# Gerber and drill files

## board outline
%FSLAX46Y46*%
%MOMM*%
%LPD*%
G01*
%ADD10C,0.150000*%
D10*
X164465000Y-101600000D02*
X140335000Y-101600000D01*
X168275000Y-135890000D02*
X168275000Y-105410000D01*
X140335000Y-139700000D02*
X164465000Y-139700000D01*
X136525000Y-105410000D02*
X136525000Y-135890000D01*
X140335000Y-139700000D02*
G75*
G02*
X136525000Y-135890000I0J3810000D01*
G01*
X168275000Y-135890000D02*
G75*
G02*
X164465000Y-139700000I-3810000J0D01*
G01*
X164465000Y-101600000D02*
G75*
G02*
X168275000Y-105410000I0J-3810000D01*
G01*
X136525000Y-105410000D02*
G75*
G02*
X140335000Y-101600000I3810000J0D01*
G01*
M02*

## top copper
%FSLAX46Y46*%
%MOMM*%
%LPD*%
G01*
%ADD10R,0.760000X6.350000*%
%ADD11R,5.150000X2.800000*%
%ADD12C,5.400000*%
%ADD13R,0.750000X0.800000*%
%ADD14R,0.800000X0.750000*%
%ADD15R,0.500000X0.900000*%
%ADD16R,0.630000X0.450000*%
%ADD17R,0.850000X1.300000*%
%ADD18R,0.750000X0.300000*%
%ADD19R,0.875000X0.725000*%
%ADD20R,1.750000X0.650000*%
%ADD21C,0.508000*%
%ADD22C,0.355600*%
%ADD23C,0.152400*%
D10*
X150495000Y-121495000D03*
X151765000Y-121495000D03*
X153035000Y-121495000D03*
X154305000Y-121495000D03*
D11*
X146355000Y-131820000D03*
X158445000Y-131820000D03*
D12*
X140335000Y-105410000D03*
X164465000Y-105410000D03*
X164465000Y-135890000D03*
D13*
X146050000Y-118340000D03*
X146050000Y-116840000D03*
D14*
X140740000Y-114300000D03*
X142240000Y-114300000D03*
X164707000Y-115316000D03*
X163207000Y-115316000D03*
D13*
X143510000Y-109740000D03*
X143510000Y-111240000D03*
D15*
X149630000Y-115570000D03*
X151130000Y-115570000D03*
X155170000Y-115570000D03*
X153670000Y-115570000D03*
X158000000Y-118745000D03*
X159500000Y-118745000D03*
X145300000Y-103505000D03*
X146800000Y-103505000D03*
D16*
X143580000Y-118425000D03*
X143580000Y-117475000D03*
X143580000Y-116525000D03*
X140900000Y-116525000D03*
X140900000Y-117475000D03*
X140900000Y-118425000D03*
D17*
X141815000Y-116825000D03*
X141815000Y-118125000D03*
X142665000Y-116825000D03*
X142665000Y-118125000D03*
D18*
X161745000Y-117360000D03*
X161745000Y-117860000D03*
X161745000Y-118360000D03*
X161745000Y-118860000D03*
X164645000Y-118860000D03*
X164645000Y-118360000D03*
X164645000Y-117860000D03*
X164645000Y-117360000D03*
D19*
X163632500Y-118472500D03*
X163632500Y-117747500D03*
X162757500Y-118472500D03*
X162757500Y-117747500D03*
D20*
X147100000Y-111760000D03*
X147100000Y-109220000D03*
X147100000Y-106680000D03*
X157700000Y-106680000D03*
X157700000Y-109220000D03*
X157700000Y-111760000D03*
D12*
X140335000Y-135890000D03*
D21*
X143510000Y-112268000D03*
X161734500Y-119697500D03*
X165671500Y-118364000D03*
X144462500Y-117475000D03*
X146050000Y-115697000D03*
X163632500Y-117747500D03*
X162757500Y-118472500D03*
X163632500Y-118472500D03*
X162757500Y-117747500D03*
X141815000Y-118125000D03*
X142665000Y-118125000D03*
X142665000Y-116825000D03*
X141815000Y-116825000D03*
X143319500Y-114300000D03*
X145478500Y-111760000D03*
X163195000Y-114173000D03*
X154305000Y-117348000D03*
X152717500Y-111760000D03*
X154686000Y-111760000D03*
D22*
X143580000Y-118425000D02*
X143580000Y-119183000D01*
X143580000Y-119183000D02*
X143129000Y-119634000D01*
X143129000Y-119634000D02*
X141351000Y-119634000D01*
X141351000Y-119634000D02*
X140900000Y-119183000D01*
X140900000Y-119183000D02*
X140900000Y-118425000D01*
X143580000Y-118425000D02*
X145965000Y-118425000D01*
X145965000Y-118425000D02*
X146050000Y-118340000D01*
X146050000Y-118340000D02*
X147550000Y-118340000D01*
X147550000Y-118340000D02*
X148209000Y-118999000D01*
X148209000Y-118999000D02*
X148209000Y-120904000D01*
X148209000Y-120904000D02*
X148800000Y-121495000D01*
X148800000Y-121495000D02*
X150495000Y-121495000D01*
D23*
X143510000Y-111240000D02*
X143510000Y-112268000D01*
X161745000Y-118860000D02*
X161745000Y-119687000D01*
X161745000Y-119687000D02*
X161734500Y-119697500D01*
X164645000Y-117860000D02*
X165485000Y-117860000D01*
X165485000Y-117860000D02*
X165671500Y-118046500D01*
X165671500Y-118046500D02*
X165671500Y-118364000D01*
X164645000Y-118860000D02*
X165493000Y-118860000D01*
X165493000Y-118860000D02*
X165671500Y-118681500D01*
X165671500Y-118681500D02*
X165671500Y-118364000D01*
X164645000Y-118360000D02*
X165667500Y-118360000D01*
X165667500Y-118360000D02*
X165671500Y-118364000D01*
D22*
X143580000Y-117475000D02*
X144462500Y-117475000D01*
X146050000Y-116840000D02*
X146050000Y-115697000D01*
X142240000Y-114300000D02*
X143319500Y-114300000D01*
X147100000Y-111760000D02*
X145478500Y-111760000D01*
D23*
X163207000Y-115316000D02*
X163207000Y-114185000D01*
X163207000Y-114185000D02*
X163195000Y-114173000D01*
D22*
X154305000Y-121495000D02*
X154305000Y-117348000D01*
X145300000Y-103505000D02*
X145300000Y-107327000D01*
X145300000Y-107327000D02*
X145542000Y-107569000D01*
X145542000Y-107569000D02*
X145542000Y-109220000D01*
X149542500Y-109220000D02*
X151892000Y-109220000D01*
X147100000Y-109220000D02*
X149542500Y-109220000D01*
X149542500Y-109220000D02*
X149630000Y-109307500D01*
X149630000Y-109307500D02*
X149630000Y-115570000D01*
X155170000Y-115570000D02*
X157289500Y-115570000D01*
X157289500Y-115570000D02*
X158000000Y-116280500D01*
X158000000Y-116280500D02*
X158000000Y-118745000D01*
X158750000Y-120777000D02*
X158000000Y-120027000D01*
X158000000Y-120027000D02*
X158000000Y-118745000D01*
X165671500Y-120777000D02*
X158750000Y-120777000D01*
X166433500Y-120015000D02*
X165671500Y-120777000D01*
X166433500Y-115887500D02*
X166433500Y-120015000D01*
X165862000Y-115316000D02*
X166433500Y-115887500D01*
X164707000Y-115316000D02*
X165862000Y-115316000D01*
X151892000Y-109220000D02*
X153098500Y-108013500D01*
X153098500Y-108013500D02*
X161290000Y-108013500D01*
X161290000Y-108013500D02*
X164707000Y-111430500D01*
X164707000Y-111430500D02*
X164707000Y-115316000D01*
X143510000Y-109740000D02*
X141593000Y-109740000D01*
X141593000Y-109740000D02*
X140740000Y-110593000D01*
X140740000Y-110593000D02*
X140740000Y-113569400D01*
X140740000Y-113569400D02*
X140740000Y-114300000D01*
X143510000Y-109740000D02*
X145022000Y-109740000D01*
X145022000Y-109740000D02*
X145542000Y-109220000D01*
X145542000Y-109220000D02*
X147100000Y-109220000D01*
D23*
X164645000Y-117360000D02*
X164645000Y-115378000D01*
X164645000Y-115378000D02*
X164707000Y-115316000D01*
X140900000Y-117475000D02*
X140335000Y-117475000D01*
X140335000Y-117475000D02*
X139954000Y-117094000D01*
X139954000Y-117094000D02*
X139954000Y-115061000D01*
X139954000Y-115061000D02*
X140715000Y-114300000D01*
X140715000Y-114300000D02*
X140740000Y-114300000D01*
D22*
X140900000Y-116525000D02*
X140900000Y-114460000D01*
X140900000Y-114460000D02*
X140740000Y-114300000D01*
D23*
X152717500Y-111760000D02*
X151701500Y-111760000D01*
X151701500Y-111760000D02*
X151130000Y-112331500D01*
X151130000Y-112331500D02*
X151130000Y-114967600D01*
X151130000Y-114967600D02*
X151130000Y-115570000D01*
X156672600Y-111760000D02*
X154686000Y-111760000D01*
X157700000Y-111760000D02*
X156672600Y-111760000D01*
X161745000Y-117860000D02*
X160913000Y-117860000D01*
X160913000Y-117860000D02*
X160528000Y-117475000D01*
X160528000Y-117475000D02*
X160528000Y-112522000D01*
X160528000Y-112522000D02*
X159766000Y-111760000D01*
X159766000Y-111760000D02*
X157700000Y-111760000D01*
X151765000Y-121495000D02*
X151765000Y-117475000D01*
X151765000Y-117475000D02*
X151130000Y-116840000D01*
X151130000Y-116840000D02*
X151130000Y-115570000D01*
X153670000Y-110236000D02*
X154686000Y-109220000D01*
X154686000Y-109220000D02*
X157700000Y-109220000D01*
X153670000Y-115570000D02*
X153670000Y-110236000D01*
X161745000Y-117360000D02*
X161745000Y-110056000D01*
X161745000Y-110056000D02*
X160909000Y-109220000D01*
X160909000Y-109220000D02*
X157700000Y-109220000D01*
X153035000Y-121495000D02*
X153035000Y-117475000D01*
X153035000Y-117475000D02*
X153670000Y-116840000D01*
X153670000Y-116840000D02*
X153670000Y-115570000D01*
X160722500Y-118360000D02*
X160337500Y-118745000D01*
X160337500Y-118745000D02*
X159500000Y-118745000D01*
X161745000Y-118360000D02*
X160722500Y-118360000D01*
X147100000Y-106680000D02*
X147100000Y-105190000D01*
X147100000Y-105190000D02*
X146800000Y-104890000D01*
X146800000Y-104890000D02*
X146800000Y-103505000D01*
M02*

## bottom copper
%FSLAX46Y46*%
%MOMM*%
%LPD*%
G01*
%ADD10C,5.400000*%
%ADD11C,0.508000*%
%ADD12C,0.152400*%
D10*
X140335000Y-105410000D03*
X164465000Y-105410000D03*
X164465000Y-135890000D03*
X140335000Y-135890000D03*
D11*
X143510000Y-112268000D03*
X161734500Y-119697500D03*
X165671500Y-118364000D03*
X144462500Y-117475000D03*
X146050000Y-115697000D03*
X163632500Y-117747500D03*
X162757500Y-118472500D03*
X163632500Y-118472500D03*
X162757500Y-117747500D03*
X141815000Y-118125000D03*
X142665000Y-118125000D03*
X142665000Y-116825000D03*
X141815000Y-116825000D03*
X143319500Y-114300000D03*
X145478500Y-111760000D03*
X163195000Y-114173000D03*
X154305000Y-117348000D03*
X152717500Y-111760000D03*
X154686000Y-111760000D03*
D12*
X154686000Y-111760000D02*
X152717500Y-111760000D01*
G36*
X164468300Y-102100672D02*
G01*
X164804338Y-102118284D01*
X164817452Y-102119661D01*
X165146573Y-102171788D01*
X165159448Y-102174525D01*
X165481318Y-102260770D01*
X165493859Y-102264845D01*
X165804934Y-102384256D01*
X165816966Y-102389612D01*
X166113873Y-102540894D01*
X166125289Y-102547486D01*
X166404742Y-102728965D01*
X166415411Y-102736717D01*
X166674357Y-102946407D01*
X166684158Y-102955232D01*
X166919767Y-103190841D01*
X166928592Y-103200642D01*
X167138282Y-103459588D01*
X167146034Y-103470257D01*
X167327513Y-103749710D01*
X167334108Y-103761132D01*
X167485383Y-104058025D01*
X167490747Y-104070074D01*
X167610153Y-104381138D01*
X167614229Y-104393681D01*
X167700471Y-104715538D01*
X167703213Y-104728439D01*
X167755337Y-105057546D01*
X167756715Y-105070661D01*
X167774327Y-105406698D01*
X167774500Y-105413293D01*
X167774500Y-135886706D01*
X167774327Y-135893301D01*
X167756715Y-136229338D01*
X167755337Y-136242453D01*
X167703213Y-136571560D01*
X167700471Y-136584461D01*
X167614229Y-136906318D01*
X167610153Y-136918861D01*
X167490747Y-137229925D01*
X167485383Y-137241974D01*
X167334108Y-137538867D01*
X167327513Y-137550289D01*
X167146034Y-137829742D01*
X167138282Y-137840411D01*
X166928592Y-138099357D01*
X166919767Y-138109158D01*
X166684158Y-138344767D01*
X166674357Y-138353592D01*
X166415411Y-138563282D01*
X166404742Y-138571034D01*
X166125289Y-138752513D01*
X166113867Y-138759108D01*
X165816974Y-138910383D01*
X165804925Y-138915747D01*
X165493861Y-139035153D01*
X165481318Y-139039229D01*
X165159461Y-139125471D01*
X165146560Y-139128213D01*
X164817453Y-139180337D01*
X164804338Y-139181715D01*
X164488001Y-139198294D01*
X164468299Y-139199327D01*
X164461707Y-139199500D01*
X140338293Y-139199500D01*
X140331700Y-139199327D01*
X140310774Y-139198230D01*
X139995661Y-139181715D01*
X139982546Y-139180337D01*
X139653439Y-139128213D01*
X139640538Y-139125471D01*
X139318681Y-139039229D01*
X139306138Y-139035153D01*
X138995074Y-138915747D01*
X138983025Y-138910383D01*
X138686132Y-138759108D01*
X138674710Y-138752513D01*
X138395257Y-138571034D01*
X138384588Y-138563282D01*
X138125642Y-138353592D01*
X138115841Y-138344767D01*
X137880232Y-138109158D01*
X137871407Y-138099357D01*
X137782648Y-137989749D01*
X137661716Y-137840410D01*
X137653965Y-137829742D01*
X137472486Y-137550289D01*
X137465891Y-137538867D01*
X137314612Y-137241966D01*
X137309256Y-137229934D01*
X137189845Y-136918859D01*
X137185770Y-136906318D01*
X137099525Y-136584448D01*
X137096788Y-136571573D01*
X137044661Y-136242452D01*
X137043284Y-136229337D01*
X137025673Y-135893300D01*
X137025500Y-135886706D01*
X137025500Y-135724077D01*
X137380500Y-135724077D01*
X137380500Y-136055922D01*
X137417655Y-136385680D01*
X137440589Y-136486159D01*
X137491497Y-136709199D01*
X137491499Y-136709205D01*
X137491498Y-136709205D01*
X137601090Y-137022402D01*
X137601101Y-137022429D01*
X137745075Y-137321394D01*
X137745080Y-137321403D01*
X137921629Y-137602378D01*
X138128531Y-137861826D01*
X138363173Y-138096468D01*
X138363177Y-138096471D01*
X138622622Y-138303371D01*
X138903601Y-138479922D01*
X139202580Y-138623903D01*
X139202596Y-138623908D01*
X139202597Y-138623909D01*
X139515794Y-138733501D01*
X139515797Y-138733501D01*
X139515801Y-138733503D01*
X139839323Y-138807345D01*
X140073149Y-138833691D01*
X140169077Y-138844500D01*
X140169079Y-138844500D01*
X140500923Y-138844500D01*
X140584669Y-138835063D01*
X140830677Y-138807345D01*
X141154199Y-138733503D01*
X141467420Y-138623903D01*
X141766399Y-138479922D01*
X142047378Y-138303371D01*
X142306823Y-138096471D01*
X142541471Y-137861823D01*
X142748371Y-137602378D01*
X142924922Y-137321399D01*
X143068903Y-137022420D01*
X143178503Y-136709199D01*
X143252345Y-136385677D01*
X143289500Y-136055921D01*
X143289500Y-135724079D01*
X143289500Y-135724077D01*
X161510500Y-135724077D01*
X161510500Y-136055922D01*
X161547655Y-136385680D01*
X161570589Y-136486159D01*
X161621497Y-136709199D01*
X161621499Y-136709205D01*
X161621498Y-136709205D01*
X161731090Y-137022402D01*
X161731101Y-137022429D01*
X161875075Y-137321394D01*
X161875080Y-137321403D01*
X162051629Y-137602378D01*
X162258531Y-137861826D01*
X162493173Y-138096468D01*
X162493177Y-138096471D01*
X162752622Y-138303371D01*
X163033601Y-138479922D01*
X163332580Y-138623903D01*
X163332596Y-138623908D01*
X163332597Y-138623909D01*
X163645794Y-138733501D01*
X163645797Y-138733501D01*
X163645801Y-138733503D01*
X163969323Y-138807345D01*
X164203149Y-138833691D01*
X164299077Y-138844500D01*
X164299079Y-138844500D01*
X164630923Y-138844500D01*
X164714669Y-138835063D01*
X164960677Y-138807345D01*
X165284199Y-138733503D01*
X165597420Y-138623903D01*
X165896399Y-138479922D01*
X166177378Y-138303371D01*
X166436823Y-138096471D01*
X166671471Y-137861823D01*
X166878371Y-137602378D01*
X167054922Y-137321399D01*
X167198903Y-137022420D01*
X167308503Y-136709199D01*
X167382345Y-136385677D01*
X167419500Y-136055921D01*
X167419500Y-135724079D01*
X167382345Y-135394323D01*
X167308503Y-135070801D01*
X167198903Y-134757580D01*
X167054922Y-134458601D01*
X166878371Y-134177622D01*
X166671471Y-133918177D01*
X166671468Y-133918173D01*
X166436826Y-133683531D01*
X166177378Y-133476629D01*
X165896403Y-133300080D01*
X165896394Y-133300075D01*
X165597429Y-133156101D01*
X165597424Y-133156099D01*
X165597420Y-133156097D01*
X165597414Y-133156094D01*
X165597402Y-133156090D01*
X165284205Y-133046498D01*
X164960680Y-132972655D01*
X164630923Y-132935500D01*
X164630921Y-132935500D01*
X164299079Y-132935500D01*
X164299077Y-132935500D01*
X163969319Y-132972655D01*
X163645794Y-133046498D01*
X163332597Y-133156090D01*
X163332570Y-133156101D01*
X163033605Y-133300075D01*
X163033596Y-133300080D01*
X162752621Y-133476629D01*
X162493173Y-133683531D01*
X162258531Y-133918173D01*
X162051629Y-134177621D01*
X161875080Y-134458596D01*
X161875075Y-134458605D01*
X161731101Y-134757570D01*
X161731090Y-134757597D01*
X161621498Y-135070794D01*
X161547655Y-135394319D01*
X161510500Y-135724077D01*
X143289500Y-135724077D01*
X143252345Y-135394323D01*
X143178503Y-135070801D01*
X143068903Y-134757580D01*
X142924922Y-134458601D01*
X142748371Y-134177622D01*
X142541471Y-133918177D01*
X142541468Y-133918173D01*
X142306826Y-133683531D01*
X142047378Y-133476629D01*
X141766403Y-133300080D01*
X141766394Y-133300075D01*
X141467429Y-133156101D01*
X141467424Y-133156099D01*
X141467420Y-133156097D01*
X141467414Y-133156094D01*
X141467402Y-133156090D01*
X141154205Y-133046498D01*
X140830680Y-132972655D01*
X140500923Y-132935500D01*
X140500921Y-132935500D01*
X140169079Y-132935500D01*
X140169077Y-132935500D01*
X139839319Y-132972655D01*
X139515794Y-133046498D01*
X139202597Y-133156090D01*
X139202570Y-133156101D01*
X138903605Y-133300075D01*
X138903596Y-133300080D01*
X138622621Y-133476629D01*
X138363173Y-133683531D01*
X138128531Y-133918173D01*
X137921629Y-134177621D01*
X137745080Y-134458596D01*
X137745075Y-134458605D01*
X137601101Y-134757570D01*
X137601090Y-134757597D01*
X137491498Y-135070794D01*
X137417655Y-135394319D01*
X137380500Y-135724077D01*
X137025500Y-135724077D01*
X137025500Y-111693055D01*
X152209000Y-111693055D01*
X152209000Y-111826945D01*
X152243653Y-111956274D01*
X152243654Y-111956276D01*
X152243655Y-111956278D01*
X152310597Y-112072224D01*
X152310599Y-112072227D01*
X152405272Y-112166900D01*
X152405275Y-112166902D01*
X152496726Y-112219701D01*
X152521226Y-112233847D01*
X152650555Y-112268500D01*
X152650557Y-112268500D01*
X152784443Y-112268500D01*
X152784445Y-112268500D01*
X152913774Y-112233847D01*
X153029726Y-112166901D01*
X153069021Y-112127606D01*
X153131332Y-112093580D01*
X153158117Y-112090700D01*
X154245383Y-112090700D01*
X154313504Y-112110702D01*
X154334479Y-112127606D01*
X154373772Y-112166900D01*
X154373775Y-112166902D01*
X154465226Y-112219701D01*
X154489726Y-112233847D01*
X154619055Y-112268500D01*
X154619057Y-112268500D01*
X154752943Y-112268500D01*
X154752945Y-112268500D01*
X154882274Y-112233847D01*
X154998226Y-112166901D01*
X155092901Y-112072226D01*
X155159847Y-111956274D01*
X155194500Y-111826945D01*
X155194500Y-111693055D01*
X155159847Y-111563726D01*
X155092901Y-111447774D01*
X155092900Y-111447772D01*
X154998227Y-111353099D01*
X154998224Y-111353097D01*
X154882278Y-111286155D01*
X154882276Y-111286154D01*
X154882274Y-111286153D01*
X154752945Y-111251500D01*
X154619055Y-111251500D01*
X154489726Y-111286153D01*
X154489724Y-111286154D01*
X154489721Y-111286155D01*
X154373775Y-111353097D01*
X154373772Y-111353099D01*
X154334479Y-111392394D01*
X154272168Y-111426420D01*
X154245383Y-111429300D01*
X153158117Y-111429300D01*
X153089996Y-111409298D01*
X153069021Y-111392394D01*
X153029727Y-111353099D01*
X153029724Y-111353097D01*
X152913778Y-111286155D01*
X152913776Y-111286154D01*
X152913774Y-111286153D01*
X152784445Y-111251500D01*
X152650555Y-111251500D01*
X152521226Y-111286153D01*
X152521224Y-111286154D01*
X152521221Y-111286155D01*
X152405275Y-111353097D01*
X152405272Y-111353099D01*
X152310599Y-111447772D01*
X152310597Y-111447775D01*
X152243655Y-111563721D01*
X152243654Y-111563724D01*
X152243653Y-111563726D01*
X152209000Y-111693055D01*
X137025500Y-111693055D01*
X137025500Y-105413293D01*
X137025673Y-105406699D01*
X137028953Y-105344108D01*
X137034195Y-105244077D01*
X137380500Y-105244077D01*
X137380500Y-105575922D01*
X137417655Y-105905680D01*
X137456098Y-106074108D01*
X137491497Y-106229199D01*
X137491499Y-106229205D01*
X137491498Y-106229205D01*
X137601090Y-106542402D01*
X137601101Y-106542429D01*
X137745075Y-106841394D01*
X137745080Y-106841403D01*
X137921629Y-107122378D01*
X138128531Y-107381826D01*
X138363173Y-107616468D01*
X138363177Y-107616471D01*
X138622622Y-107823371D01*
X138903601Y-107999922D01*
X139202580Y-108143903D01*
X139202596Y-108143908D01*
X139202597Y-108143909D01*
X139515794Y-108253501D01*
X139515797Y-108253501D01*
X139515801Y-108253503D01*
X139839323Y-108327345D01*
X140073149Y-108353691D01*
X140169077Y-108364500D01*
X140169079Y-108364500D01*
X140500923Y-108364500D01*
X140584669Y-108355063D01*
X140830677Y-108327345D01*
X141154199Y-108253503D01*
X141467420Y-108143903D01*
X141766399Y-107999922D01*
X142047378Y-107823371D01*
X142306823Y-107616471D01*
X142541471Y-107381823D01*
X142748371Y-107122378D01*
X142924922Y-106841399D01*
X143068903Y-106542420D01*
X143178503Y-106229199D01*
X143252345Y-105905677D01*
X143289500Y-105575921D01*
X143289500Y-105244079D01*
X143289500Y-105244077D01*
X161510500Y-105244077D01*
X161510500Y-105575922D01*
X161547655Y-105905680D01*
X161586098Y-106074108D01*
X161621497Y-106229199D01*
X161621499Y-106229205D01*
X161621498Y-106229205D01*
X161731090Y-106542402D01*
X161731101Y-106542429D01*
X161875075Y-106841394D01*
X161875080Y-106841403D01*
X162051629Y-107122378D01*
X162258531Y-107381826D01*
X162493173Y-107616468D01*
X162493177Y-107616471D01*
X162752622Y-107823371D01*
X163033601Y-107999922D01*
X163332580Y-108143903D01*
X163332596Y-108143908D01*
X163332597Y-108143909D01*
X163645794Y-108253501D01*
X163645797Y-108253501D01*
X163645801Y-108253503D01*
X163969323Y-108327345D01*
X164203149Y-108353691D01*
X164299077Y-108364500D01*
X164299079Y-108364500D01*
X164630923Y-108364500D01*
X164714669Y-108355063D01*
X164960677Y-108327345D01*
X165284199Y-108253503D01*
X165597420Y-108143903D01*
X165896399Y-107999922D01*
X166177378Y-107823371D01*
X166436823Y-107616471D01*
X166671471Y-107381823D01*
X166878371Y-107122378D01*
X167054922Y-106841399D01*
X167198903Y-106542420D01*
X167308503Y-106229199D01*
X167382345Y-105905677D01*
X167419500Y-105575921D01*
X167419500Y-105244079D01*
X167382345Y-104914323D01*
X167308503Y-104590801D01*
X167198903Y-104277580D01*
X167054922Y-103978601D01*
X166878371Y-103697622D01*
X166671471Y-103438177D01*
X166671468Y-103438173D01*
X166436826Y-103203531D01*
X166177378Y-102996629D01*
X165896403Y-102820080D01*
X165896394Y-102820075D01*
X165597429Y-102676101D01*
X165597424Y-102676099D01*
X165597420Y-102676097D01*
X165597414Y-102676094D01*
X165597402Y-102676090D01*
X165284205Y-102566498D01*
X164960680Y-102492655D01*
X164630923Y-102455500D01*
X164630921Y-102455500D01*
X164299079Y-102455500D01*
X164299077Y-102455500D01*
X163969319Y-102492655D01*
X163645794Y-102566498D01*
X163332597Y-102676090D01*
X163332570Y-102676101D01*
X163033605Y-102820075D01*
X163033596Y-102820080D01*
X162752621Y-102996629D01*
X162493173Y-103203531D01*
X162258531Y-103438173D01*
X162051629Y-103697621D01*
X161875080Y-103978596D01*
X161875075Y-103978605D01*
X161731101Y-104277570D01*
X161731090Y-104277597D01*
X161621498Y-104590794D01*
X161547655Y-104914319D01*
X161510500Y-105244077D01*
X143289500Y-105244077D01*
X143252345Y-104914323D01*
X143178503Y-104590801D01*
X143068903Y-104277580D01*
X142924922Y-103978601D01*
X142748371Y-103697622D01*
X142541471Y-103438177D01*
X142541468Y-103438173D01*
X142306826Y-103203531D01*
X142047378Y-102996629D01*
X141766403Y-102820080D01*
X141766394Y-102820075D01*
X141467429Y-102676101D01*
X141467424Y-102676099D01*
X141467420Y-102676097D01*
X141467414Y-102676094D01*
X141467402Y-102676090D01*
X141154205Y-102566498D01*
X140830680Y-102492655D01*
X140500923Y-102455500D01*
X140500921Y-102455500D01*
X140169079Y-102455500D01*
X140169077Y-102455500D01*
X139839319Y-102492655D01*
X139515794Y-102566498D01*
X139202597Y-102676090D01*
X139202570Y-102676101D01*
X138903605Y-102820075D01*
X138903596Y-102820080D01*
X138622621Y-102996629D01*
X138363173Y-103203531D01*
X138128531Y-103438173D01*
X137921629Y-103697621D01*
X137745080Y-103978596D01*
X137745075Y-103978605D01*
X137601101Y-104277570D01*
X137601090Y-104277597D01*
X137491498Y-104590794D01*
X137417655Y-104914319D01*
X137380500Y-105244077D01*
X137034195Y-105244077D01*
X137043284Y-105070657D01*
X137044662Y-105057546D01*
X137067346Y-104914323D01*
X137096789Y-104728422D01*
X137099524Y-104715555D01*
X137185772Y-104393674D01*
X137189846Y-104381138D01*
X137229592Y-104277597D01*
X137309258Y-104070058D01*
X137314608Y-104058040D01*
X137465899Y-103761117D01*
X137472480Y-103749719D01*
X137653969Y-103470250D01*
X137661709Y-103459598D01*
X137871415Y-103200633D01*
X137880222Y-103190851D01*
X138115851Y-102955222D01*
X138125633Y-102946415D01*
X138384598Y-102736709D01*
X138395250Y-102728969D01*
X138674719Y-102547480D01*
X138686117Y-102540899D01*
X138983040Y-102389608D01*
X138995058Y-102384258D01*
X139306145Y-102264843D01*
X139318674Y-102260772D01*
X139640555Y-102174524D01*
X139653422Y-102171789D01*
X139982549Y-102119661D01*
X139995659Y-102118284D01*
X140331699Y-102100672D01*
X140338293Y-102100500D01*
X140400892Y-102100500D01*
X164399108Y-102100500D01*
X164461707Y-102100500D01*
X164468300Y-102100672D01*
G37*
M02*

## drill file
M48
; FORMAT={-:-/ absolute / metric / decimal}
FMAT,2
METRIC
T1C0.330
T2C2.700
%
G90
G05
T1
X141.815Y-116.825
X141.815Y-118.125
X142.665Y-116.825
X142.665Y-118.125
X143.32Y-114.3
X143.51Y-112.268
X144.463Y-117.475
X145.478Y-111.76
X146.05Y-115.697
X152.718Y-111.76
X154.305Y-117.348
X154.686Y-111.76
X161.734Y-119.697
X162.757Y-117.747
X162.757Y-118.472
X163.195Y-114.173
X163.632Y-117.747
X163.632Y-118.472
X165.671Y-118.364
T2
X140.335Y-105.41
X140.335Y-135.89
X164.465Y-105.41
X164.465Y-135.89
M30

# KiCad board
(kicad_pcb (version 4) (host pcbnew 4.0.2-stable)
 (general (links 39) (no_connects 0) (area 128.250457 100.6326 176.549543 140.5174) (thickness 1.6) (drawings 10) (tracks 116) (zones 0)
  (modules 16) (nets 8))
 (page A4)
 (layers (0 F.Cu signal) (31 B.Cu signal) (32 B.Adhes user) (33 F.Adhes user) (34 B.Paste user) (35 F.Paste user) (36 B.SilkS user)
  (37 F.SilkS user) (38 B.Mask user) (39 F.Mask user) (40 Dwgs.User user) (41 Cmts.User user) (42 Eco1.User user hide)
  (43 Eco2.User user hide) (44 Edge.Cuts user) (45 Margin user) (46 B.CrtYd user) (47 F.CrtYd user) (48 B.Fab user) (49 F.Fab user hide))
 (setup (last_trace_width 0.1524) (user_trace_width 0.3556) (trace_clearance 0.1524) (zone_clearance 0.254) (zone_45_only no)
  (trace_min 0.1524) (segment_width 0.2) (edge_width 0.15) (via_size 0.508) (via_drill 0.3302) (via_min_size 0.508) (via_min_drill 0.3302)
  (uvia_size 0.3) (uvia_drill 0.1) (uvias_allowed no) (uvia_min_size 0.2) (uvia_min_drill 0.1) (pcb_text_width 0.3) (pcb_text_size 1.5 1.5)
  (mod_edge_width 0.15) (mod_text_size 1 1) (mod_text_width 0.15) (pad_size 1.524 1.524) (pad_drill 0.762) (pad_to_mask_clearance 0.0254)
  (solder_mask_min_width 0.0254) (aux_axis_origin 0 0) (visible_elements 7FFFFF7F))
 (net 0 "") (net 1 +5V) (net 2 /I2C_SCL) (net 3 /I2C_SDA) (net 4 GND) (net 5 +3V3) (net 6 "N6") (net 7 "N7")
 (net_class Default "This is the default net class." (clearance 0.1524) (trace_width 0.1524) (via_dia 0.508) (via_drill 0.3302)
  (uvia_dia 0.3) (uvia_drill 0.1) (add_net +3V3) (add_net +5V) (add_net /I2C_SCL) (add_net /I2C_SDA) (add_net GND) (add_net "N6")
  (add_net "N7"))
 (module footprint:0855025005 (layer F.Cu) (at 152.4 139.7)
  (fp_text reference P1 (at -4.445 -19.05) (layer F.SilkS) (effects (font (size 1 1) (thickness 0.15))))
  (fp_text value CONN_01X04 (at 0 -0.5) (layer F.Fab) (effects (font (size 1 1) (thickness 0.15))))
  (pad 1 smd rect (at -1.905 -18.205) (size 0.76 6.35) (layers F.Cu F.Paste F.Mask) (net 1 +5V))
  (pad 2 smd rect (at -0.635 -18.205) (size 0.76 6.35) (layers F.Cu F.Paste F.Mask) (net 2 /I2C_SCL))
  (pad 3 smd rect (at 0.635 -18.205) (size 0.76 6.35) (layers F.Cu F.Paste F.Mask) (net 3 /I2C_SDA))
  (pad 4 smd rect (at 1.905 -18.205) (size 0.76 6.35) (layers F.Cu F.Paste F.Mask) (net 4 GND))
  (pad 5 smd rect (at -6.045 -7.88) (size 5.15 2.8) (layers F.Cu F.Paste F.Mask))
  (pad 5 smd rect (at 6.045 -7.88) (size 5.15 2.8) (layers F.Cu F.Paste F.Mask)))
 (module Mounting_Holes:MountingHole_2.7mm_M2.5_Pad (layer F.Cu) (at 140.335 105.41)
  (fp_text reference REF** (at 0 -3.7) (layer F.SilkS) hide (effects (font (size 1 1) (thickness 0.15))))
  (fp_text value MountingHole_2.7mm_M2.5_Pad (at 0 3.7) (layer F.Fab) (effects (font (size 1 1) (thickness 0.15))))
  (pad 1 thru_hole circle (at 0 0) (size 5.4 5.4) (drill 2.7) (layers *.Cu *.Mask F.SilkS)))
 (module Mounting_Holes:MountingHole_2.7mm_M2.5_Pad (layer F.Cu) (at 164.465 105.41)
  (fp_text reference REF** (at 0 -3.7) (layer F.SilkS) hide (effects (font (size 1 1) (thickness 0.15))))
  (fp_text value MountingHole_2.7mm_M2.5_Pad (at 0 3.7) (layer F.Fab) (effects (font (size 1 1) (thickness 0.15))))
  (pad 1 thru_hole circle (at 0 0) (size 5.4 5.4) (drill 2.7) (layers *.Cu *.Mask F.SilkS)))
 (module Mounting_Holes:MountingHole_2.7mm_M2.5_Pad (layer F.Cu) (at 164.465 135.89)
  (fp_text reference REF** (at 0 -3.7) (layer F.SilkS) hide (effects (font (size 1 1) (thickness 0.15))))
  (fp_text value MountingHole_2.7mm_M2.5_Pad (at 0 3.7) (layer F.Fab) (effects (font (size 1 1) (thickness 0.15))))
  (pad 1 thru_hole circle (at 0 0) (size 5.4 5.4) (drill 2.7) (layers *.Cu *.Mask F.SilkS)))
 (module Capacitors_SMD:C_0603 (layer F.Cu) (at 146.05 117.59 90)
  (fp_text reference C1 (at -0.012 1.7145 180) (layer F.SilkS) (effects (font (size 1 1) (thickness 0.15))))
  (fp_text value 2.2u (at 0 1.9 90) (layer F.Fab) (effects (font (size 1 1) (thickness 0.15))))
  (pad 1 smd rect (at -0.75 0 90) (size 0.8 0.75) (layers F.Cu F.Paste F.Mask) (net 1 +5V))
  (pad 2 smd rect (at 0.75 0 90) (size 0.8 0.75) (layers F.Cu F.Paste F.Mask) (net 4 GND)))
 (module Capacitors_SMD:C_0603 (layer F.Cu) (at 141.49 114.3)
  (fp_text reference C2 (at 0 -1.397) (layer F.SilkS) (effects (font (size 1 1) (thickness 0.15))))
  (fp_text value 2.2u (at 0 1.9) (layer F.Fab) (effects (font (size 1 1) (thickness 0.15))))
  (pad 1 smd rect (at -0.75 0) (size 0.8 0.75) (layers F.Cu F.Paste F.Mask) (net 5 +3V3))
  (pad 2 smd rect (at 0.75 0) (size 0.8 0.75) (layers F.Cu F.Paste F.Mask) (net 4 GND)))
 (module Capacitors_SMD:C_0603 (layer F.Cu) (at 163.957 115.316 180)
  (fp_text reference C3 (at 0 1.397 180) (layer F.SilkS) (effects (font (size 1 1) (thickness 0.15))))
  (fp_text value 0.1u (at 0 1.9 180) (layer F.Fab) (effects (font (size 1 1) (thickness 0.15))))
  (pad 1 smd rect (at -0.75 0 180) (size 0.8 0.75) (layers F.Cu F.Paste F.Mask) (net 5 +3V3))
  (pad 2 smd rect (at 0.75 0 180) (size 0.8 0.75) (layers F.Cu F.Paste F.Mask) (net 4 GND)))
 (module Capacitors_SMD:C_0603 (layer F.Cu) (at 143.51 110.49 270)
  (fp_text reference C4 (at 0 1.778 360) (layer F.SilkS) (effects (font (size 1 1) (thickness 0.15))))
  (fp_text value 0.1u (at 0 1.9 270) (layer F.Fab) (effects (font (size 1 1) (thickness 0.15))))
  (pad 1 smd rect (at -0.75 0 270) (size 0.8 0.75) (layers F.Cu F.Paste F.Mask) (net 5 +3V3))
  (pad 2 smd rect (at 0.75 0 270) (size 0.8 0.75) (layers F.Cu F.Paste F.Mask) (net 4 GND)))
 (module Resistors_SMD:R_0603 (layer F.Cu) (at 150.38 115.57)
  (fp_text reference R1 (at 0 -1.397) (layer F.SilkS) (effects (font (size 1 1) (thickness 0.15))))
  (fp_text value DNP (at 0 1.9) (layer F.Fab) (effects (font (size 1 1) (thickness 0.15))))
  (pad 1 smd rect (at -0.75 0) (size 0.5 0.9) (layers F.Cu F.Paste F.Mask) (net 5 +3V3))
  (pad 2 smd rect (at 0.75 0) (size 0.5 0.9) (layers F.Cu F.Paste F.Mask) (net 2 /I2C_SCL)))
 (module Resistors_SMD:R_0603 (layer F.Cu) (at 154.42 115.57 180)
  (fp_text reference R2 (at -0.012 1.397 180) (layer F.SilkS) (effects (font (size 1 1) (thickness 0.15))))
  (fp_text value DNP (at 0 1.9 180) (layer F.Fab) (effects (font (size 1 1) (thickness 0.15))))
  (pad 1 smd rect (at -0.75 0 180) (size 0.5 0.9) (layers F.Cu F.Paste F.Mask) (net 5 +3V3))
  (pad 2 smd rect (at 0.75 0 180) (size 0.5 0.9) (layers F.Cu F.Paste F.Mask) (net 3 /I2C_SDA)))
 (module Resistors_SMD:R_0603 (layer F.Cu) (at 158.75 118.745)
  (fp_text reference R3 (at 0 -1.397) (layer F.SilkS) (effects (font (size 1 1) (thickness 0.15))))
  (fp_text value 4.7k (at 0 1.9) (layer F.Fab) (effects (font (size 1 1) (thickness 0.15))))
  (pad 1 smd rect (at -0.75 0) (size 0.5 0.9) (layers F.Cu F.Paste F.Mask) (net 5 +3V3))
  (pad 2 smd rect (at 0.75 0) (size 0.5 0.9) (layers F.Cu F.Paste F.Mask) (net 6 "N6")))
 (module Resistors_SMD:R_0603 (layer F.Cu) (at 146.05 103.505)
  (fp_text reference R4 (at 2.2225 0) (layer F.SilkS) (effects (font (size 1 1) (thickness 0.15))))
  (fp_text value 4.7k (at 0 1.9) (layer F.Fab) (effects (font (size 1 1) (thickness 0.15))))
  (pad 1 smd rect (at -0.75 0) (size 0.5 0.9) (layers F.Cu F.Paste F.Mask) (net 5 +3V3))
  (pad 2 smd rect (at 0.75 0) (size 0.5 0.9) (layers F.Cu F.Paste F.Mask) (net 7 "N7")))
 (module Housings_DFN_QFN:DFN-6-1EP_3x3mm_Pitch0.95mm (layer F.Cu) (at 142.24 117.475 180)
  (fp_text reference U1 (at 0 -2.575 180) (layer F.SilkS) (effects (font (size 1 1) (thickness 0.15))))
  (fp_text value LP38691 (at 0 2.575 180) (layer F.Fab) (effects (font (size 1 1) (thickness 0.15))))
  (pad 1 smd rect (at -1.34 -0.95 180) (size 0.63 0.45) (layers F.Cu F.Paste F.Mask) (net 1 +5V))
  (pad 2 smd rect (at -1.34 0 180) (size 0.63 0.45) (layers F.Cu F.Paste F.Mask) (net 4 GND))
  (pad 3 smd rect (at -1.34 0.95 180) (size 0.63 0.45) (layers F.Cu F.Paste F.Mask))
  (pad 4 smd rect (at 1.34 0.95 180) (size 0.63 0.45) (layers F.Cu F.Paste F.Mask) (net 5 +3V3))
  (pad 5 smd rect (at 1.34 0 180) (size 0.63 0.45) (layers F.Cu F.Paste F.Mask) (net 5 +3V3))
  (pad 6 smd rect (at 1.34 -0.95 180) (size 0.63 0.45) (layers F.Cu F.Paste F.Mask) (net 1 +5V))
  (pad 7 smd rect (at 0.425 0.65 180) (size 0.85 1.3) (layers F.Cu F.Paste F.Mask) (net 4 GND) (solder_paste_margin_ratio -0.2))
  (pad 7 smd rect (at 0.425 -0.65 180) (size 0.85 1.3) (layers F.Cu F.Paste F.Mask) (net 4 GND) (solder_paste_margin_ratio -0.2))
  (pad 7 smd rect (at -0.425 0.65 180) (size 0.85 1.3) (layers F.Cu F.Paste F.Mask) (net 4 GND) (solder_paste_margin_ratio -0.2))
  (pad 7 smd rect (at -0.425 -0.65 180) (size 0.85 1.3) (layers F.Cu F.Paste F.Mask) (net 4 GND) (solder_paste_margin_ratio -0.2)))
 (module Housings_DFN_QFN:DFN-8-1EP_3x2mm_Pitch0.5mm (layer F.Cu) (at 163.195 118.11)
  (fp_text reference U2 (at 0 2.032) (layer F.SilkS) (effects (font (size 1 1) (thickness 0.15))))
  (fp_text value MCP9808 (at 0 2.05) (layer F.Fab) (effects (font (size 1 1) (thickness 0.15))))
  (pad 1 smd rect (at -1.45 -0.75) (size 0.75 0.3) (layers F.Cu F.Paste F.Mask) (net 3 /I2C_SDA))
  (pad 2 smd rect (at -1.45 -0.25) (size 0.75 0.3) (layers F.Cu F.Paste F.Mask) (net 2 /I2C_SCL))
  (pad 3 smd rect (at -1.45 0.25) (size 0.75 0.3) (layers F.Cu F.Paste F.Mask) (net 6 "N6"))
  (pad 4 smd rect (at -1.45 0.75) (size 0.75 0.3) (layers F.Cu F.Paste F.Mask) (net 4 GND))
  (pad 5 smd rect (at 1.45 0.75) (size 0.75 0.3) (layers F.Cu F.Paste F.Mask) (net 4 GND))
  (pad 6 smd rect (at 1.45 0.25) (size 0.75 0.3) (layers F.Cu F.Paste F.Mask) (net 4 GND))
  (pad 7 smd rect (at 1.45 -0.25) (size 0.75 0.3) (layers F.Cu F.Paste F.Mask) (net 4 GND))
  (pad 8 smd rect (at 1.45 -0.75) (size 0.75 0.3) (layers F.Cu F.Paste F.Mask) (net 5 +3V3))
  (pad 9 smd rect (at 0.4375 0.3625) (size 0.875 0.725) (layers F.Cu F.Paste F.Mask) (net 4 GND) (solder_paste_margin_ratio -0.2))
  (pad 9 smd rect (at 0.4375 -0.3625) (size 0.875 0.725) (layers F.Cu F.Paste F.Mask) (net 4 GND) (solder_paste_margin_ratio -0.2))
  (pad 9 smd rect (at -0.4375 0.3625) (size 0.875 0.725) (layers F.Cu F.Paste F.Mask) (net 4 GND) (solder_paste_margin_ratio -0.2))
  (pad 9 smd rect (at -0.4375 -0.3625) (size 0.875 0.725) (layers F.Cu F.Paste F.Mask) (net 4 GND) (solder_paste_margin_ratio -0.2)))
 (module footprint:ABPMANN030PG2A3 (layer F.Cu) (at 152.4 109.22)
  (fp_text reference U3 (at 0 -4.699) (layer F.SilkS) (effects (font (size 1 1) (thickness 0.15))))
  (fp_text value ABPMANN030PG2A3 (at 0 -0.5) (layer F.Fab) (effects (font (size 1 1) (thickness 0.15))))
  (pad 1 smd rect (at -5.3 2.54) (size 1.75 0.65) (layers F.Cu F.Paste F.Mask) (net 4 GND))
  (pad 2 smd rect (at -5.3 0) (size 1.75 0.65) (layers F.Cu F.Paste F.Mask) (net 5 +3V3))
  (pad 3 smd rect (at -5.3 -2.54) (size 1.75 0.65) (layers F.Cu F.Paste F.Mask) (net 7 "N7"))
  (pad 4 smd rect (at 5.3 -2.54) (size 1.75 0.65) (layers F.Cu F.Paste F.Mask))
  (pad 5 smd rect (at 5.3 0) (size 1.75 0.65) (layers F.Cu F.Paste F.Mask) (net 3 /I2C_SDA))
  (pad 6 smd rect (at 5.3 2.54) (size 1.75 0.65) (layers F.Cu F.Paste F.Mask) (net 2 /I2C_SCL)))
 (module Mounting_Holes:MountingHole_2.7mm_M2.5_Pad (layer F.Cu) (at 140.335 135.89)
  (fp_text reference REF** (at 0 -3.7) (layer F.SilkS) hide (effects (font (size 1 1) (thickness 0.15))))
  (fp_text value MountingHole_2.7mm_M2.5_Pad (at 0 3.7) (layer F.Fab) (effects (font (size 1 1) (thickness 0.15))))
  (pad 1 thru_hole circle (at 0 0) (size 5.4 5.4) (drill 2.7) (layers *.Cu *.Mask F.SilkS)))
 (gr_line (start 164.465 101.6) (end 140.335 101.6) (layer Edge.Cuts) (width 0.15))
 (gr_line (start 168.275 135.89) (end 168.275 105.41) (layer Edge.Cuts) (width 0.15))
 (gr_line (start 140.335 139.7) (end 164.465 139.7) (layer Edge.Cuts) (width 0.15))
 (gr_line (start 136.525 105.41) (end 136.525 135.89) (layer Edge.Cuts) (width 0.15))
 (gr_arc (start 140.335 135.89) (end 140.335 139.7) (angle 90) (layer Edge.Cuts) (width 0.15))
 (gr_arc (start 164.465 135.89) (end 168.275 135.89) (angle 90) (layer Edge.Cuts) (width 0.15))
 (gr_arc (start 164.465 105.41) (end 164.465 101.6) (angle 90) (layer Edge.Cuts) (width 0.15))
 (gr_arc (start 140.335 105.41) (end 136.525 105.41) (angle 90) (layer Edge.Cuts) (width 0.15))
 (segment (start 143.58 118.425) (end 143.58 119.183) (width 0.3556) (layer F.Cu) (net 1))
 (segment (start 143.58 119.183) (end 143.129 119.634) (width 0.3556) (layer F.Cu) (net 1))
 (segment (start 143.129 119.634) (end 141.351 119.634) (width 0.3556) (layer F.Cu) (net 1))
 (segment (start 141.351 119.634) (end 140.9 119.183) (width 0.3556) (layer F.Cu) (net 1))
 (segment (start 140.9 119.183) (end 140.9 118.425) (width 0.3556) (layer F.Cu) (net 1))
 (segment (start 143.58 118.425) (end 145.965 118.425) (width 0.3556) (layer F.Cu) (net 1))
 (segment (start 145.965 118.425) (end 146.05 118.34) (width 0.3556) (layer F.Cu) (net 1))
 (segment (start 146.05 118.34) (end 147.55 118.34) (width 0.3556) (layer F.Cu) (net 1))
 (segment (start 147.55 118.34) (end 148.209 118.999) (width 0.3556) (layer F.Cu) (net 1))
 (segment (start 148.209 118.999) (end 148.209 120.904) (width 0.3556) (layer F.Cu) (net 1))
 (segment (start 148.209 120.904) (end 148.8 121.495) (width 0.3556) (layer F.Cu) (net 1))
 (segment (start 148.8 121.495) (end 150.495 121.495) (width 0.3556) (layer F.Cu) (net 1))
 (segment (start 143.51 111.24) (end 143.51 112.268) (width 0.1524) (layer F.Cu) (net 4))
 (via (at 143.51 112.268) (size 0.508) (drill 0.3302) (layers F.Cu B.Cu) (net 4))
 (segment (start 161.745 118.86) (end 161.745 119.687) (width 0.1524) (layer F.Cu) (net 4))
 (segment (start 161.745 119.687) (end 161.7345 119.6975) (width 0.1524) (layer F.Cu) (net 4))
 (via (at 161.7345 119.6975) (size 0.508) (drill 0.3302) (layers F.Cu B.Cu) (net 4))
 (segment (start 164.645 117.86) (end 165.485 117.86) (width 0.1524) (layer F.Cu) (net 4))
 (segment (start 165.485 117.86) (end 165.6715 118.0465) (width 0.1524) (layer F.Cu) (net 4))
 (segment (start 165.6715 118.0465) (end 165.6715 118.364) (width 0.1524) (layer F.Cu) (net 4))
 (segment (start 164.645 118.86) (end 165.493 118.86) (width 0.1524) (layer F.Cu) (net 4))
 (segment (start 165.493 118.86) (end 165.6715 118.6815) (width 0.1524) (layer F.Cu) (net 4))
 (segment (start 165.6715 118.6815) (end 165.6715 118.364) (width 0.1524) (layer F.Cu) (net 4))
 (segment (start 164.645 118.36) (end 165.6675 118.36) (width 0.1524) (layer F.Cu) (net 4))
 (segment (start 165.6675 118.36) (end 165.6715 118.364) (width 0.1524) (layer F.Cu) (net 4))
 (via (at 165.6715 118.364) (size 0.508) (drill 0.3302) (layers F.Cu B.Cu) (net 4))
 (segment (start 143.58 117.475) (end 144.4625 117.475) (width 0.3556) (layer F.Cu) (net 4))
 (via (at 144.4625 117.475) (size 0.508) (drill 0.3302) (layers F.Cu B.Cu) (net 4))
 (segment (start 146.05 116.84) (end 146.05 115.697) (width 0.3556) (layer F.Cu) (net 4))
 (via (at 146.05 115.697) (size 0.508) (drill 0.3302) (layers F.Cu B.Cu) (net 4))
 (via (at 163.6325 117.7475) (size 0.508) (drill 0.3302) (layers F.Cu B.Cu) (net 4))
 (via (at 162.7575 118.4725) (size 0.508) (drill 0.3302) (layers F.Cu B.Cu) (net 4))
 (via (at 163.6325 118.4725) (size 0.508) (drill 0.3302) (layers F.Cu B.Cu) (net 4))
 (via (at 162.7575 117.7475) (size 0.508) (drill 0.3302) (layers F.Cu B.Cu) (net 4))
 (via (at 141.815 118.125) (size 0.508) (drill 0.3302) (layers F.Cu B.Cu) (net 4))
 (via (at 142.665 118.125) (size 0.508) (drill 0.3302) (layers F.Cu B.Cu) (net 4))
 (via (at 142.665 116.825) (size 0.508) (drill 0.3302) (layers F.Cu B.Cu) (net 4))
 (via (at 141.815 116.825) (size 0.508) (drill 0.3302) (layers F.Cu B.Cu) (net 4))
 (segment (start 142.24 114.3) (end 143.3195 114.3) (width 0.3556) (layer F.Cu) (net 4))
 (via (at 143.3195 114.3) (size 0.508) (drill 0.3302) (layers F.Cu B.Cu) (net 4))
 (segment (start 147.1 111.76) (end 145.4785 111.76) (width 0.3556) (layer F.Cu) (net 4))
 (via (at 145.4785 111.76) (size 0.508) (drill 0.3302) (layers F.Cu B.Cu) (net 4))
 (segment (start 163.207 115.316) (end 163.207 114.185) (width 0.1524) (layer F.Cu) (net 4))
 (segment (start 163.207 114.185) (end 163.195 114.173) (width 0.1524) (layer F.Cu) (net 4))
 (via (at 163.195 114.173) (size 0.508) (drill 0.3302) (layers F.Cu B.Cu) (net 4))
 (segment (start 154.305 121.495) (end 154.305 117.348) (width 0.3556) (layer F.Cu) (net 4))
 (via (at 154.305 117.348) (size 0.508) (drill 0.3302) (layers F.Cu B.Cu) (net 4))
 (segment (start 145.3 103.505) (end 145.3 107.327) (width 0.3556) (layer F.Cu) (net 5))
 (segment (start 145.3 107.327) (end 145.542 107.569) (width 0.3556) (layer F.Cu) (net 5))
 (segment (start 145.542 107.569) (end 145.542 109.22) (width 0.3556) (layer F.Cu) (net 5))
 (segment (start 149.5425 109.22) (end 151.892 109.22) (width 0.3556) (layer F.Cu) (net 5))
 (segment (start 147.1 109.22) (end 149.5425 109.22) (width 0.3556) (layer F.Cu) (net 5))
 (segment (start 149.5425 109.22) (end 149.63 109.3075) (width 0.3556) (layer F.Cu) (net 5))
 (segment (start 149.63 109.3075) (end 149.63 115.57) (width 0.3556) (layer F.Cu) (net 5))
 (segment (start 155.17 115.57) (end 157.2895 115.57) (width 0.3556) (layer F.Cu) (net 5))
 (segment (start 157.2895 115.57) (end 158 116.2805) (width 0.3556) (layer F.Cu) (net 5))
 (segment (start 158 116.2805) (end 158 118.745) (width 0.3556) (layer F.Cu) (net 5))
 (segment (start 158.75 120.777) (end 158 120.027) (width 0.3556) (layer F.Cu) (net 5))
 (segment (start 158 120.027) (end 158 118.745) (width 0.3556) (layer F.Cu) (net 5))
 (segment (start 165.6715 120.777) (end 158.75 120.777) (width 0.3556) (layer F.Cu) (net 5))
 (segment (start 166.4335 120.015) (end 165.6715 120.777) (width 0.3556) (layer F.Cu) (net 5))
 (segment (start 166.4335 115.8875) (end 166.4335 120.015) (width 0.3556) (layer F.Cu) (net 5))
 (segment (start 165.862 115.316) (end 166.4335 115.8875) (width 0.3556) (layer F.Cu) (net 5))
 (segment (start 164.707 115.316) (end 165.862 115.316) (width 0.3556) (layer F.Cu) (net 5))
 (segment (start 151.892 109.22) (end 153.0985 108.0135) (width 0.3556) (layer F.Cu) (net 5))
 (segment (start 153.0985 108.0135) (end 161.29 108.0135) (width 0.3556) (layer F.Cu) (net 5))
 (segment (start 161.29 108.0135) (end 164.707 111.4305) (width 0.3556) (layer F.Cu) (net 5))
 (segment (start 164.707 111.4305) (end 164.707 115.316) (width 0.3556) (layer F.Cu) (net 5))
 (segment (start 143.51 109.74) (end 141.593 109.74) (width 0.3556) (layer F.Cu) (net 5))
 (segment (start 141.593 109.74) (end 140.74 110.593) (width 0.3556) (layer F.Cu) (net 5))
 (segment (start 140.74 110.593) (end 140.74 113.5694) (width 0.3556) (layer F.Cu) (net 5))
 (segment (start 140.74 113.5694) (end 140.74 114.3) (width 0.3556) (layer F.Cu) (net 5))
 (segment (start 143.51 109.74) (end 145.022 109.74) (width 0.3556) (layer F.Cu) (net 5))
 (segment (start 145.022 109.74) (end 145.542 109.22) (width 0.3556) (layer F.Cu) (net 5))
 (segment (start 145.542 109.22) (end 147.1 109.22) (width 0.3556) (layer F.Cu) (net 5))
 (segment (start 164.645 117.36) (end 164.645 115.378) (width 0.1524) (layer F.Cu) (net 5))
 (segment (start 164.645 115.378) (end 164.707 115.316) (width 0.1524) (layer F.Cu) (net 5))
 (segment (start 140.9 117.475) (end 140.335 117.475) (width 0.1524) (layer F.Cu) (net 5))
 (segment (start 140.335 117.475) (end 139.954 117.094) (width 0.1524) (layer F.Cu) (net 5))
 (segment (start 139.954 117.094) (end 139.954 115.061) (width 0.1524) (layer F.Cu) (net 5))
 (segment (start 139.954 115.061) (end 140.715 114.3) (width 0.1524) (layer F.Cu) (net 5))
 (segment (start 140.715 114.3) (end 140.74 114.3) (width 0.1524) (layer F.Cu) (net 5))
 (segment (start 140.9 116.525) (end 140.9 114.46) (width 0.3556) (layer F.Cu) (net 5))
 (segment (start 140.9 114.46) (end 140.74 114.3) (width 0.3556) (layer F.Cu) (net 5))
 (segment (start 152.7175 111.76) (end 151.7015 111.76) (width 0.1524) (layer F.Cu) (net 2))
 (segment (start 151.7015 111.76) (end 151.13 112.3315) (width 0.1524) (layer F.Cu) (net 2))
 (segment (start 151.13 112.3315) (end 151.13 114.9676) (width 0.1524) (layer F.Cu) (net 2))
 (segment (start 151.13 114.9676) (end 151.13 115.57) (width 0.1524) (layer F.Cu) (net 2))
 (segment (start 154.686 111.76) (end 152.7175 111.76) (width 0.1524) (layer B.Cu) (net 2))
 (via (at 152.7175 111.76) (size 0.508) (drill 0.3302) (layers F.Cu B.Cu) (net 2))
 (segment (start 156.6726 111.76) (end 154.686 111.76) (width 0.1524) (layer F.Cu) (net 2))
 (via (at 154.686 111.76) (size 0.508) (drill 0.3302) (layers F.Cu B.Cu) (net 2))
 (segment (start 157.7 111.76) (end 156.6726 111.76) (width 0.1524) (layer F.Cu) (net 2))
 (segment (start 161.745 117.86) (end 160.913 117.86) (width 0.1524) (layer F.Cu) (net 2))
 (segment (start 160.913 117.86) (end 160.528 117.475) (width 0.1524) (layer F.Cu) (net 2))
 (segment (start 160.528 117.475) (end 160.528 112.522) (width 0.1524) (layer F.Cu) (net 2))
 (segment (start 160.528 112.522) (end 159.766 111.76) (width 0.1524) (layer F.Cu) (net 2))
 (segment (start 159.766 111.76) (end 157.7 111.76) (width 0.1524) (layer F.Cu) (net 2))
 (segment (start 151.765 121.495) (end 151.765 117.475) (width 0.1524) (layer F.Cu) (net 2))
 (segment (start 151.765 117.475) (end 151.13 116.84) (width 0.1524) (layer F.Cu) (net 2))
 (segment (start 151.13 116.84) (end 151.13 115.57) (width 0.1524) (layer F.Cu) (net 2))
 (segment (start 153.67 110.236) (end 154.686 109.22) (width 0.1524) (layer F.Cu) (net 3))
 (segment (start 154.686 109.22) (end 157.7 109.22) (width 0.1524) (layer F.Cu) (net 3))
 (segment (start 153.67 115.57) (end 153.67 110.236) (width 0.1524) (layer F.Cu) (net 3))
 (segment (start 161.745 117.36) (end 161.745 110.056) (width 0.1524) (layer F.Cu) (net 3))
 (segment (start 161.745 110.056) (end 160.909 109.22) (width 0.1524) (layer F.Cu) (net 3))
 (segment (start 160.909 109.22) (end 157.7 109.22) (width 0.1524) (layer F.Cu) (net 3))
 (segment (start 153.035 121.495) (end 153.035 117.475) (width 0.1524) (layer F.Cu) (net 3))
 (segment (start 153.035 117.475) (end 153.67 116.84) (width 0.1524) (layer F.Cu) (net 3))
 (segment (start 153.67 116.84) (end 153.67 115.57) (width 0.1524) (layer F.Cu) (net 3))
 (segment (start 160.7225 118.36) (end 160.3375 118.745) (width 0.1524) (layer F.Cu) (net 6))
 (segment (start 160.3375 118.745) (end 159.5 118.745) (width 0.1524) (layer F.Cu) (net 6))
 (segment (start 161.745 118.36) (end 160.7225 118.36) (width 0.1524) (layer F.Cu) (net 6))
 (segment (start 147.1 106.68) (end 147.1 105.19) (width 0.1524) (layer F.Cu) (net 7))
 (segment (start 147.1 105.19) (end 146.8 104.89) (width 0.1524) (layer F.Cu) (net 7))
 (segment (start 146.8 104.89) (end 146.8 103.505) (width 0.1524) (layer F.Cu) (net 7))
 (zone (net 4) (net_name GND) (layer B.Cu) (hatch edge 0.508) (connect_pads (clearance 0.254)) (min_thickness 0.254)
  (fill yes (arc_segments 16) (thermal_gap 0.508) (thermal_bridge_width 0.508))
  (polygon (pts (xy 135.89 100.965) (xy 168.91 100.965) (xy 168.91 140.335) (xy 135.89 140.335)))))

